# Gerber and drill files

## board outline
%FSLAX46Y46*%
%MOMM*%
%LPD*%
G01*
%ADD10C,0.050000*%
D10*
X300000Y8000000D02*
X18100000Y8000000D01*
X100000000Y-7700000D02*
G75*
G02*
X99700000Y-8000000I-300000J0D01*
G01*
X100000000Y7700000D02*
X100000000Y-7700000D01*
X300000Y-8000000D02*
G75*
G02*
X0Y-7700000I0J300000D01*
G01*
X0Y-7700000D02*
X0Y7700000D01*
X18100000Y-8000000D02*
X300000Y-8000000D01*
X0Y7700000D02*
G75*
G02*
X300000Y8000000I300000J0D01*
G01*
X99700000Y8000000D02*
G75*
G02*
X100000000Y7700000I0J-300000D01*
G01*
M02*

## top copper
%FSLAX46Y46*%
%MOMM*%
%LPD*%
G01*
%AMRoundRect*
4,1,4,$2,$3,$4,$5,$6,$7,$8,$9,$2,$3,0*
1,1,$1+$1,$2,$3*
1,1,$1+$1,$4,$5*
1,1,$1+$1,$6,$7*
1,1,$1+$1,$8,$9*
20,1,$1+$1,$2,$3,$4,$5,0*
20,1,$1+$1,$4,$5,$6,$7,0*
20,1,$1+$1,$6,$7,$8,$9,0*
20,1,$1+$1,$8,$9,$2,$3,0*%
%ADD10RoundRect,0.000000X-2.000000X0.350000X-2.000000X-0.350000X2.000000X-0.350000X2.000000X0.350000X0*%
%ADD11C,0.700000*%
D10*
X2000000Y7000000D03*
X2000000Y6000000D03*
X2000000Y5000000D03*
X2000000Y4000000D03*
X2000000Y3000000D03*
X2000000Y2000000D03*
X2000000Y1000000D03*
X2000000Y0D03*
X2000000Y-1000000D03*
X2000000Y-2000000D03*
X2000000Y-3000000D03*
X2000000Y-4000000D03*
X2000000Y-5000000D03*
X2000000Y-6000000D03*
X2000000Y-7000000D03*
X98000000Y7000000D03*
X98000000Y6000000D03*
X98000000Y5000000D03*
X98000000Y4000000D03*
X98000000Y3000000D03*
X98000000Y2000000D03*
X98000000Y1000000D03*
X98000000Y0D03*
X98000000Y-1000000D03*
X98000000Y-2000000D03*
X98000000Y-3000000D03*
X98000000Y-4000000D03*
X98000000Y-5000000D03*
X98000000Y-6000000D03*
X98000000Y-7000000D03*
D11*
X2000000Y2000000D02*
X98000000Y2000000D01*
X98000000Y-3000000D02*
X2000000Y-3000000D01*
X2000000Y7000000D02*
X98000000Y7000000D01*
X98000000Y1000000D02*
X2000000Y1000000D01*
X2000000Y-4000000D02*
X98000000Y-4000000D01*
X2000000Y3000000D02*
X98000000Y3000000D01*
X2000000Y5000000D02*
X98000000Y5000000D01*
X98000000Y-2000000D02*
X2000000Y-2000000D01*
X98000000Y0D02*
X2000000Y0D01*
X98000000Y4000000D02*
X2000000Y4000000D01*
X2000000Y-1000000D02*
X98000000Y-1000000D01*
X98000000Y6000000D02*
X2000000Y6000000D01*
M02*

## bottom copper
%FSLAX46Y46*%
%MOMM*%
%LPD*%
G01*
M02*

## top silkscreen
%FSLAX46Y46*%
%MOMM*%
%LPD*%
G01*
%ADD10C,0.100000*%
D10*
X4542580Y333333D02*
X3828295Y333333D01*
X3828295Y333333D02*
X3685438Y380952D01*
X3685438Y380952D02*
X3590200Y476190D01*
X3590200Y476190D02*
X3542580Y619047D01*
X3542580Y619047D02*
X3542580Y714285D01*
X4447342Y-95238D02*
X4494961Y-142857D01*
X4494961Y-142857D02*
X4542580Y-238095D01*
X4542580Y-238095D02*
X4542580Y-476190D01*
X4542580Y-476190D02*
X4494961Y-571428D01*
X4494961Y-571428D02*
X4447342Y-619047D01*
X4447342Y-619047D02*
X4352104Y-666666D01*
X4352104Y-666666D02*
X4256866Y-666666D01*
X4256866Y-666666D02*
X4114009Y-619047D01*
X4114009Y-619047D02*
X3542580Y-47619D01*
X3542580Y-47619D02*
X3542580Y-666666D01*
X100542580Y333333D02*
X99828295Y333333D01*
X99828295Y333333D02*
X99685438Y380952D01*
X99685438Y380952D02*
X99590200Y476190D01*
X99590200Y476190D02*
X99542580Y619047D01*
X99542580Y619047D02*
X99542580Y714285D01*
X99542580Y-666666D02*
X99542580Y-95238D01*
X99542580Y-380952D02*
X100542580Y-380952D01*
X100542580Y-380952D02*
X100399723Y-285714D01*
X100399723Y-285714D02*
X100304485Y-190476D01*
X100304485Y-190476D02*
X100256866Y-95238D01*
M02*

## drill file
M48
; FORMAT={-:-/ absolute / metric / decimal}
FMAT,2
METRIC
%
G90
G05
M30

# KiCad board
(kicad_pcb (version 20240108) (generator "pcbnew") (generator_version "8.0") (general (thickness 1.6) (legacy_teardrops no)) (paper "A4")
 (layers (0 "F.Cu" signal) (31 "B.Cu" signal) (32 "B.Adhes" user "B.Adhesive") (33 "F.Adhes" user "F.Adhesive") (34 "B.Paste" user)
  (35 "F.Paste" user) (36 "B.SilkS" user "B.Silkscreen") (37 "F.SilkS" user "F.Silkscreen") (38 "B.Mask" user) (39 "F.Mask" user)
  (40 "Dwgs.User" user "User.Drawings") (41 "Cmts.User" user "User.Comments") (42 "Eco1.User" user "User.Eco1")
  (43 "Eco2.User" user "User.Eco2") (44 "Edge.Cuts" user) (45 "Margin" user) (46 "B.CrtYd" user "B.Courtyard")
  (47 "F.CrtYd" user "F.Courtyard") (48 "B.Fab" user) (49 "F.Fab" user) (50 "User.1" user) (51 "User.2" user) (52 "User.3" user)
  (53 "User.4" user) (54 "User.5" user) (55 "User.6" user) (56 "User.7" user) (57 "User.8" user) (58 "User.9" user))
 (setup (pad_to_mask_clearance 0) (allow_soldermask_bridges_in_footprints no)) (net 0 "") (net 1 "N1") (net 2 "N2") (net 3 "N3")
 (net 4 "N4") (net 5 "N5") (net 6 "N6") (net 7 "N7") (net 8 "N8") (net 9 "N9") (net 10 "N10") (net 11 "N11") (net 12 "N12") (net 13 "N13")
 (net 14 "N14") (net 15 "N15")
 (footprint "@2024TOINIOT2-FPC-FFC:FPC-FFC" (layer "F.Cu") (at 2 0 -90)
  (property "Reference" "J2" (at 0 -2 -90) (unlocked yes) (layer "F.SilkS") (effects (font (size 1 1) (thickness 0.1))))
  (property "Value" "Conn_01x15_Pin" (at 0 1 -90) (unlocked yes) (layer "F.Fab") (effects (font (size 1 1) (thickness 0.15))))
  (pad "1" smd roundrect (at -7 0 270) (size 0.7 4) (layers "F.Cu" "F.Paste" "B.SilkS" "F.Mask") (roundrect_rratio 0) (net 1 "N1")
   (thermal_bridge_angle 45))
  (pad "2" smd roundrect (at -6 0 270) (size 0.7 4) (layers "F.Cu" "F.Paste" "B.SilkS" "F.Mask") (roundrect_rratio 0) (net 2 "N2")
   (thermal_bridge_angle 45))
  (pad "3" smd roundrect (at -5 0 270) (size 0.7 4) (layers "F.Cu" "F.Paste" "B.SilkS" "F.Mask") (roundrect_rratio 0) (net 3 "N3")
   (thermal_bridge_angle 45))
  (pad "4" smd roundrect (at -4 0 270) (size 0.7 4) (layers "F.Cu" "F.Paste" "B.SilkS" "F.Mask") (roundrect_rratio 0) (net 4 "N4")
   (thermal_bridge_angle 45))
  (pad "5" smd roundrect (at -3 0 270) (size 0.7 4) (layers "F.Cu" "F.Paste" "B.SilkS" "F.Mask") (roundrect_rratio 0) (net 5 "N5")
   (thermal_bridge_angle 45))
  (pad "6" smd roundrect (at -2 0 270) (size 0.7 4) (layers "F.Cu" "F.Paste" "B.SilkS" "F.Mask") (roundrect_rratio 0) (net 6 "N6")
   (thermal_bridge_angle 45))
  (pad "7" smd roundrect (at -1 0 270) (size 0.7 4) (layers "F.Cu" "F.Paste" "B.SilkS" "F.Mask") (roundrect_rratio 0) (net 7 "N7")
   (thermal_bridge_angle 45))
  (pad "8" smd roundrect (at 0 0 270) (size 0.7 4) (layers "F.Cu" "F.Paste" "B.SilkS" "F.Mask") (roundrect_rratio 0) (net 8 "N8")
   (thermal_bridge_angle 45))
  (pad "9" smd roundrect (at 1 0 270) (size 0.7 4) (layers "F.Cu" "F.Paste" "B.SilkS" "F.Mask") (roundrect_rratio 0) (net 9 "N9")
   (thermal_bridge_angle 45))
  (pad "10" smd roundrect (at 2 0 270) (size 0.7 4) (layers "F.Cu" "F.Paste" "B.SilkS" "F.Mask") (roundrect_rratio 0) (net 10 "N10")
   (thermal_bridge_angle 45))
  (pad "11" smd roundrect (at 3 0 270) (size 0.7 4) (layers "F.Cu" "F.Paste" "B.SilkS" "F.Mask") (roundrect_rratio 0) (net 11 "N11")
   (thermal_bridge_angle 45))
  (pad "12" smd roundrect (at 4 0 270) (size 0.7 4) (layers "F.Cu" "F.Paste" "B.SilkS" "F.Mask") (roundrect_rratio 0) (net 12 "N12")
   (thermal_bridge_angle 45))
  (pad "13" smd roundrect (at 5 0 270) (size 0.7 4) (layers "F.Cu" "F.Paste" "B.SilkS" "F.Mask") (roundrect_rratio 0) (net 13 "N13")
   (thermal_bridge_angle 45))
  (pad "14" smd roundrect (at 6 0 270) (size 0.7 4) (layers "F.Cu" "F.Paste" "B.SilkS" "F.Mask") (roundrect_rratio 0) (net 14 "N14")
   (thermal_bridge_angle 45))
  (pad "15" smd roundrect (at 7 0 270) (size 0.7 4) (layers "F.Cu" "F.Paste" "B.SilkS" "F.Mask") (roundrect_rratio 0) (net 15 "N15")
   (thermal_bridge_angle 45)))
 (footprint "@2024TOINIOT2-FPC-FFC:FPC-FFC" (layer "F.Cu") (at 98 0 -90)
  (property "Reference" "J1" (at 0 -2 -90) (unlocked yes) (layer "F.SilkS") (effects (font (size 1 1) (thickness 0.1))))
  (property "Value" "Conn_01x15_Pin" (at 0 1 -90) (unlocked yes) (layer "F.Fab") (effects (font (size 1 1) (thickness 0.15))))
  (pad "1" smd roundrect (at -7 0 270) (size 0.7 4) (layers "F.Cu" "F.Paste" "B.SilkS" "F.Mask") (roundrect_rratio 0) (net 1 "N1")
   (thermal_bridge_angle 45))
  (pad "2" smd roundrect (at -6 0 270) (size 0.7 4) (layers "F.Cu" "F.Paste" "B.SilkS" "F.Mask") (roundrect_rratio 0) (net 2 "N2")
   (thermal_bridge_angle 45))
  (pad "3" smd roundrect (at -5 0 270) (size 0.7 4) (layers "F.Cu" "F.Paste" "B.SilkS" "F.Mask") (roundrect_rratio 0) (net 3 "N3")
   (thermal_bridge_angle 45))
  (pad "4" smd roundrect (at -4 0 270) (size 0.7 4) (layers "F.Cu" "F.Paste" "B.SilkS" "F.Mask") (roundrect_rratio 0) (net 4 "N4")
   (thermal_bridge_angle 45))
  (pad "5" smd roundrect (at -3 0 270) (size 0.7 4) (layers "F.Cu" "F.Paste" "B.SilkS" "F.Mask") (roundrect_rratio 0) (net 5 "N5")
   (thermal_bridge_angle 45))
  (pad "6" smd roundrect (at -2 0 270) (size 0.7 4) (layers "F.Cu" "F.Paste" "B.SilkS" "F.Mask") (roundrect_rratio 0) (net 6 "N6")
   (thermal_bridge_angle 45))
  (pad "7" smd roundrect (at -1 0 270) (size 0.7 4) (layers "F.Cu" "F.Paste" "B.SilkS" "F.Mask") (roundrect_rratio 0) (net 7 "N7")
   (thermal_bridge_angle 45))
  (pad "8" smd roundrect (at 0 0 270) (size 0.7 4) (layers "F.Cu" "F.Paste" "B.SilkS" "F.Mask") (roundrect_rratio 0) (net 8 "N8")
   (thermal_bridge_angle 45))
  (pad "9" smd roundrect (at 1 0 270) (size 0.7 4) (layers "F.Cu" "F.Paste" "B.SilkS" "F.Mask") (roundrect_rratio 0) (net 9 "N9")
   (thermal_bridge_angle 45))
  (pad "10" smd roundrect (at 2 0 270) (size 0.7 4) (layers "F.Cu" "F.Paste" "B.SilkS" "F.Mask") (roundrect_rratio 0) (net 10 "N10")
   (thermal_bridge_angle 45))
  (pad "11" smd roundrect (at 3 0 270) (size 0.7 4) (layers "F.Cu" "F.Paste" "B.SilkS" "F.Mask") (roundrect_rratio 0) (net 11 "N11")
   (thermal_bridge_angle 45))
  (pad "12" smd roundrect (at 4 0 270) (size 0.7 4) (layers "F.Cu" "F.Paste" "B.SilkS" "F.Mask") (roundrect_rratio 0) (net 12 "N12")
   (thermal_bridge_angle 45))
  (pad "13" smd roundrect (at 5 0 270) (size 0.7 4) (layers "F.Cu" "F.Paste" "B.SilkS" "F.Mask") (roundrect_rratio 0) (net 13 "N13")
   (thermal_bridge_angle 45))
  (pad "14" smd roundrect (at 6 0 270) (size 0.7 4) (layers "F.Cu" "F.Paste" "B.SilkS" "F.Mask") (roundrect_rratio 0) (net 14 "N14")
   (thermal_bridge_angle 45))
  (pad "15" smd roundrect (at 7 0 270) (size 0.7 4) (layers "F.Cu" "F.Paste" "B.SilkS" "F.Mask") (roundrect_rratio 0) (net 15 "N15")
   (thermal_bridge_angle 45)))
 (gr_line (start 0.3 -8) (end 18.1 -8) (stroke (width 0.05) (type default)) (layer "Edge.Cuts"))
 (gr_arc (start 100 7.7) (mid 99.912132 7.912132) (end 99.7 8) (stroke (width 0.05) (type default)) (layer "Edge.Cuts"))
 (gr_line (start 100 -7.7) (end 100 7.7) (stroke (width 0.05) (type default)) (layer "Edge.Cuts"))
 (gr_arc (start 0.3 8) (mid 0.087868 7.912132) (end 0 7.7) (stroke (width 0.05) (type default)) (layer "Edge.Cuts"))
 (gr_line (start 0 7.7) (end 0 -7.7) (stroke (width 0.05) (type default)) (layer "Edge.Cuts"))
 (gr_line (start 18.1 8) (end 0.3 8) (stroke (width 0.05) (type default)) (layer "Edge.Cuts"))
 (gr_arc (start 0 -7.7) (mid 0.087868 -7.912132) (end 0.3 -8) (stroke (width 0.05) (type default)) (layer "Edge.Cuts"))
 (gr_arc (start 99.7 -8) (mid 99.912132 -7.912132) (end 100 -7.7) (stroke (width 0.05) (type default)) (layer "Edge.Cuts"))
 (segment (start 2 -2) (end 98 -2) (width 0.7) (layer "F.Cu") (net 6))
 (segment (start 98 3) (end 2 3) (width 0.7) (layer "F.Cu") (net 11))
 (segment (start 2 -7) (end 98 -7) (width 0.7) (layer "F.Cu") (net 1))
 (segment (start 98 -1) (end 2 -1) (width 0.7) (layer "F.Cu") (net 7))
 (segment (start 2 4) (end 98 4) (width 0.7) (layer "F.Cu") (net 12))
 (segment (start 2 -3) (end 98 -3) (width 0.7) (layer "F.Cu") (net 5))
 (segment (start 2 -5) (end 98 -5) (width 0.7) (layer "F.Cu") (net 3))
 (segment (start 98 2) (end 2 2) (width 0.7) (layer "F.Cu") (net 10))
 (segment (start 98 0) (end 2 0) (width 0.7) (layer "F.Cu") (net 8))
 (segment (start 98 -4) (end 2 -4) (width 0.7) (layer "F.Cu") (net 4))
 (segment (start 2 1) (end 98 1) (width 0.7) (layer "F.Cu") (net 9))
 (segment (start 98 -6) (end 2 -6) (width 0.7) (layer "F.Cu") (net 2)))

